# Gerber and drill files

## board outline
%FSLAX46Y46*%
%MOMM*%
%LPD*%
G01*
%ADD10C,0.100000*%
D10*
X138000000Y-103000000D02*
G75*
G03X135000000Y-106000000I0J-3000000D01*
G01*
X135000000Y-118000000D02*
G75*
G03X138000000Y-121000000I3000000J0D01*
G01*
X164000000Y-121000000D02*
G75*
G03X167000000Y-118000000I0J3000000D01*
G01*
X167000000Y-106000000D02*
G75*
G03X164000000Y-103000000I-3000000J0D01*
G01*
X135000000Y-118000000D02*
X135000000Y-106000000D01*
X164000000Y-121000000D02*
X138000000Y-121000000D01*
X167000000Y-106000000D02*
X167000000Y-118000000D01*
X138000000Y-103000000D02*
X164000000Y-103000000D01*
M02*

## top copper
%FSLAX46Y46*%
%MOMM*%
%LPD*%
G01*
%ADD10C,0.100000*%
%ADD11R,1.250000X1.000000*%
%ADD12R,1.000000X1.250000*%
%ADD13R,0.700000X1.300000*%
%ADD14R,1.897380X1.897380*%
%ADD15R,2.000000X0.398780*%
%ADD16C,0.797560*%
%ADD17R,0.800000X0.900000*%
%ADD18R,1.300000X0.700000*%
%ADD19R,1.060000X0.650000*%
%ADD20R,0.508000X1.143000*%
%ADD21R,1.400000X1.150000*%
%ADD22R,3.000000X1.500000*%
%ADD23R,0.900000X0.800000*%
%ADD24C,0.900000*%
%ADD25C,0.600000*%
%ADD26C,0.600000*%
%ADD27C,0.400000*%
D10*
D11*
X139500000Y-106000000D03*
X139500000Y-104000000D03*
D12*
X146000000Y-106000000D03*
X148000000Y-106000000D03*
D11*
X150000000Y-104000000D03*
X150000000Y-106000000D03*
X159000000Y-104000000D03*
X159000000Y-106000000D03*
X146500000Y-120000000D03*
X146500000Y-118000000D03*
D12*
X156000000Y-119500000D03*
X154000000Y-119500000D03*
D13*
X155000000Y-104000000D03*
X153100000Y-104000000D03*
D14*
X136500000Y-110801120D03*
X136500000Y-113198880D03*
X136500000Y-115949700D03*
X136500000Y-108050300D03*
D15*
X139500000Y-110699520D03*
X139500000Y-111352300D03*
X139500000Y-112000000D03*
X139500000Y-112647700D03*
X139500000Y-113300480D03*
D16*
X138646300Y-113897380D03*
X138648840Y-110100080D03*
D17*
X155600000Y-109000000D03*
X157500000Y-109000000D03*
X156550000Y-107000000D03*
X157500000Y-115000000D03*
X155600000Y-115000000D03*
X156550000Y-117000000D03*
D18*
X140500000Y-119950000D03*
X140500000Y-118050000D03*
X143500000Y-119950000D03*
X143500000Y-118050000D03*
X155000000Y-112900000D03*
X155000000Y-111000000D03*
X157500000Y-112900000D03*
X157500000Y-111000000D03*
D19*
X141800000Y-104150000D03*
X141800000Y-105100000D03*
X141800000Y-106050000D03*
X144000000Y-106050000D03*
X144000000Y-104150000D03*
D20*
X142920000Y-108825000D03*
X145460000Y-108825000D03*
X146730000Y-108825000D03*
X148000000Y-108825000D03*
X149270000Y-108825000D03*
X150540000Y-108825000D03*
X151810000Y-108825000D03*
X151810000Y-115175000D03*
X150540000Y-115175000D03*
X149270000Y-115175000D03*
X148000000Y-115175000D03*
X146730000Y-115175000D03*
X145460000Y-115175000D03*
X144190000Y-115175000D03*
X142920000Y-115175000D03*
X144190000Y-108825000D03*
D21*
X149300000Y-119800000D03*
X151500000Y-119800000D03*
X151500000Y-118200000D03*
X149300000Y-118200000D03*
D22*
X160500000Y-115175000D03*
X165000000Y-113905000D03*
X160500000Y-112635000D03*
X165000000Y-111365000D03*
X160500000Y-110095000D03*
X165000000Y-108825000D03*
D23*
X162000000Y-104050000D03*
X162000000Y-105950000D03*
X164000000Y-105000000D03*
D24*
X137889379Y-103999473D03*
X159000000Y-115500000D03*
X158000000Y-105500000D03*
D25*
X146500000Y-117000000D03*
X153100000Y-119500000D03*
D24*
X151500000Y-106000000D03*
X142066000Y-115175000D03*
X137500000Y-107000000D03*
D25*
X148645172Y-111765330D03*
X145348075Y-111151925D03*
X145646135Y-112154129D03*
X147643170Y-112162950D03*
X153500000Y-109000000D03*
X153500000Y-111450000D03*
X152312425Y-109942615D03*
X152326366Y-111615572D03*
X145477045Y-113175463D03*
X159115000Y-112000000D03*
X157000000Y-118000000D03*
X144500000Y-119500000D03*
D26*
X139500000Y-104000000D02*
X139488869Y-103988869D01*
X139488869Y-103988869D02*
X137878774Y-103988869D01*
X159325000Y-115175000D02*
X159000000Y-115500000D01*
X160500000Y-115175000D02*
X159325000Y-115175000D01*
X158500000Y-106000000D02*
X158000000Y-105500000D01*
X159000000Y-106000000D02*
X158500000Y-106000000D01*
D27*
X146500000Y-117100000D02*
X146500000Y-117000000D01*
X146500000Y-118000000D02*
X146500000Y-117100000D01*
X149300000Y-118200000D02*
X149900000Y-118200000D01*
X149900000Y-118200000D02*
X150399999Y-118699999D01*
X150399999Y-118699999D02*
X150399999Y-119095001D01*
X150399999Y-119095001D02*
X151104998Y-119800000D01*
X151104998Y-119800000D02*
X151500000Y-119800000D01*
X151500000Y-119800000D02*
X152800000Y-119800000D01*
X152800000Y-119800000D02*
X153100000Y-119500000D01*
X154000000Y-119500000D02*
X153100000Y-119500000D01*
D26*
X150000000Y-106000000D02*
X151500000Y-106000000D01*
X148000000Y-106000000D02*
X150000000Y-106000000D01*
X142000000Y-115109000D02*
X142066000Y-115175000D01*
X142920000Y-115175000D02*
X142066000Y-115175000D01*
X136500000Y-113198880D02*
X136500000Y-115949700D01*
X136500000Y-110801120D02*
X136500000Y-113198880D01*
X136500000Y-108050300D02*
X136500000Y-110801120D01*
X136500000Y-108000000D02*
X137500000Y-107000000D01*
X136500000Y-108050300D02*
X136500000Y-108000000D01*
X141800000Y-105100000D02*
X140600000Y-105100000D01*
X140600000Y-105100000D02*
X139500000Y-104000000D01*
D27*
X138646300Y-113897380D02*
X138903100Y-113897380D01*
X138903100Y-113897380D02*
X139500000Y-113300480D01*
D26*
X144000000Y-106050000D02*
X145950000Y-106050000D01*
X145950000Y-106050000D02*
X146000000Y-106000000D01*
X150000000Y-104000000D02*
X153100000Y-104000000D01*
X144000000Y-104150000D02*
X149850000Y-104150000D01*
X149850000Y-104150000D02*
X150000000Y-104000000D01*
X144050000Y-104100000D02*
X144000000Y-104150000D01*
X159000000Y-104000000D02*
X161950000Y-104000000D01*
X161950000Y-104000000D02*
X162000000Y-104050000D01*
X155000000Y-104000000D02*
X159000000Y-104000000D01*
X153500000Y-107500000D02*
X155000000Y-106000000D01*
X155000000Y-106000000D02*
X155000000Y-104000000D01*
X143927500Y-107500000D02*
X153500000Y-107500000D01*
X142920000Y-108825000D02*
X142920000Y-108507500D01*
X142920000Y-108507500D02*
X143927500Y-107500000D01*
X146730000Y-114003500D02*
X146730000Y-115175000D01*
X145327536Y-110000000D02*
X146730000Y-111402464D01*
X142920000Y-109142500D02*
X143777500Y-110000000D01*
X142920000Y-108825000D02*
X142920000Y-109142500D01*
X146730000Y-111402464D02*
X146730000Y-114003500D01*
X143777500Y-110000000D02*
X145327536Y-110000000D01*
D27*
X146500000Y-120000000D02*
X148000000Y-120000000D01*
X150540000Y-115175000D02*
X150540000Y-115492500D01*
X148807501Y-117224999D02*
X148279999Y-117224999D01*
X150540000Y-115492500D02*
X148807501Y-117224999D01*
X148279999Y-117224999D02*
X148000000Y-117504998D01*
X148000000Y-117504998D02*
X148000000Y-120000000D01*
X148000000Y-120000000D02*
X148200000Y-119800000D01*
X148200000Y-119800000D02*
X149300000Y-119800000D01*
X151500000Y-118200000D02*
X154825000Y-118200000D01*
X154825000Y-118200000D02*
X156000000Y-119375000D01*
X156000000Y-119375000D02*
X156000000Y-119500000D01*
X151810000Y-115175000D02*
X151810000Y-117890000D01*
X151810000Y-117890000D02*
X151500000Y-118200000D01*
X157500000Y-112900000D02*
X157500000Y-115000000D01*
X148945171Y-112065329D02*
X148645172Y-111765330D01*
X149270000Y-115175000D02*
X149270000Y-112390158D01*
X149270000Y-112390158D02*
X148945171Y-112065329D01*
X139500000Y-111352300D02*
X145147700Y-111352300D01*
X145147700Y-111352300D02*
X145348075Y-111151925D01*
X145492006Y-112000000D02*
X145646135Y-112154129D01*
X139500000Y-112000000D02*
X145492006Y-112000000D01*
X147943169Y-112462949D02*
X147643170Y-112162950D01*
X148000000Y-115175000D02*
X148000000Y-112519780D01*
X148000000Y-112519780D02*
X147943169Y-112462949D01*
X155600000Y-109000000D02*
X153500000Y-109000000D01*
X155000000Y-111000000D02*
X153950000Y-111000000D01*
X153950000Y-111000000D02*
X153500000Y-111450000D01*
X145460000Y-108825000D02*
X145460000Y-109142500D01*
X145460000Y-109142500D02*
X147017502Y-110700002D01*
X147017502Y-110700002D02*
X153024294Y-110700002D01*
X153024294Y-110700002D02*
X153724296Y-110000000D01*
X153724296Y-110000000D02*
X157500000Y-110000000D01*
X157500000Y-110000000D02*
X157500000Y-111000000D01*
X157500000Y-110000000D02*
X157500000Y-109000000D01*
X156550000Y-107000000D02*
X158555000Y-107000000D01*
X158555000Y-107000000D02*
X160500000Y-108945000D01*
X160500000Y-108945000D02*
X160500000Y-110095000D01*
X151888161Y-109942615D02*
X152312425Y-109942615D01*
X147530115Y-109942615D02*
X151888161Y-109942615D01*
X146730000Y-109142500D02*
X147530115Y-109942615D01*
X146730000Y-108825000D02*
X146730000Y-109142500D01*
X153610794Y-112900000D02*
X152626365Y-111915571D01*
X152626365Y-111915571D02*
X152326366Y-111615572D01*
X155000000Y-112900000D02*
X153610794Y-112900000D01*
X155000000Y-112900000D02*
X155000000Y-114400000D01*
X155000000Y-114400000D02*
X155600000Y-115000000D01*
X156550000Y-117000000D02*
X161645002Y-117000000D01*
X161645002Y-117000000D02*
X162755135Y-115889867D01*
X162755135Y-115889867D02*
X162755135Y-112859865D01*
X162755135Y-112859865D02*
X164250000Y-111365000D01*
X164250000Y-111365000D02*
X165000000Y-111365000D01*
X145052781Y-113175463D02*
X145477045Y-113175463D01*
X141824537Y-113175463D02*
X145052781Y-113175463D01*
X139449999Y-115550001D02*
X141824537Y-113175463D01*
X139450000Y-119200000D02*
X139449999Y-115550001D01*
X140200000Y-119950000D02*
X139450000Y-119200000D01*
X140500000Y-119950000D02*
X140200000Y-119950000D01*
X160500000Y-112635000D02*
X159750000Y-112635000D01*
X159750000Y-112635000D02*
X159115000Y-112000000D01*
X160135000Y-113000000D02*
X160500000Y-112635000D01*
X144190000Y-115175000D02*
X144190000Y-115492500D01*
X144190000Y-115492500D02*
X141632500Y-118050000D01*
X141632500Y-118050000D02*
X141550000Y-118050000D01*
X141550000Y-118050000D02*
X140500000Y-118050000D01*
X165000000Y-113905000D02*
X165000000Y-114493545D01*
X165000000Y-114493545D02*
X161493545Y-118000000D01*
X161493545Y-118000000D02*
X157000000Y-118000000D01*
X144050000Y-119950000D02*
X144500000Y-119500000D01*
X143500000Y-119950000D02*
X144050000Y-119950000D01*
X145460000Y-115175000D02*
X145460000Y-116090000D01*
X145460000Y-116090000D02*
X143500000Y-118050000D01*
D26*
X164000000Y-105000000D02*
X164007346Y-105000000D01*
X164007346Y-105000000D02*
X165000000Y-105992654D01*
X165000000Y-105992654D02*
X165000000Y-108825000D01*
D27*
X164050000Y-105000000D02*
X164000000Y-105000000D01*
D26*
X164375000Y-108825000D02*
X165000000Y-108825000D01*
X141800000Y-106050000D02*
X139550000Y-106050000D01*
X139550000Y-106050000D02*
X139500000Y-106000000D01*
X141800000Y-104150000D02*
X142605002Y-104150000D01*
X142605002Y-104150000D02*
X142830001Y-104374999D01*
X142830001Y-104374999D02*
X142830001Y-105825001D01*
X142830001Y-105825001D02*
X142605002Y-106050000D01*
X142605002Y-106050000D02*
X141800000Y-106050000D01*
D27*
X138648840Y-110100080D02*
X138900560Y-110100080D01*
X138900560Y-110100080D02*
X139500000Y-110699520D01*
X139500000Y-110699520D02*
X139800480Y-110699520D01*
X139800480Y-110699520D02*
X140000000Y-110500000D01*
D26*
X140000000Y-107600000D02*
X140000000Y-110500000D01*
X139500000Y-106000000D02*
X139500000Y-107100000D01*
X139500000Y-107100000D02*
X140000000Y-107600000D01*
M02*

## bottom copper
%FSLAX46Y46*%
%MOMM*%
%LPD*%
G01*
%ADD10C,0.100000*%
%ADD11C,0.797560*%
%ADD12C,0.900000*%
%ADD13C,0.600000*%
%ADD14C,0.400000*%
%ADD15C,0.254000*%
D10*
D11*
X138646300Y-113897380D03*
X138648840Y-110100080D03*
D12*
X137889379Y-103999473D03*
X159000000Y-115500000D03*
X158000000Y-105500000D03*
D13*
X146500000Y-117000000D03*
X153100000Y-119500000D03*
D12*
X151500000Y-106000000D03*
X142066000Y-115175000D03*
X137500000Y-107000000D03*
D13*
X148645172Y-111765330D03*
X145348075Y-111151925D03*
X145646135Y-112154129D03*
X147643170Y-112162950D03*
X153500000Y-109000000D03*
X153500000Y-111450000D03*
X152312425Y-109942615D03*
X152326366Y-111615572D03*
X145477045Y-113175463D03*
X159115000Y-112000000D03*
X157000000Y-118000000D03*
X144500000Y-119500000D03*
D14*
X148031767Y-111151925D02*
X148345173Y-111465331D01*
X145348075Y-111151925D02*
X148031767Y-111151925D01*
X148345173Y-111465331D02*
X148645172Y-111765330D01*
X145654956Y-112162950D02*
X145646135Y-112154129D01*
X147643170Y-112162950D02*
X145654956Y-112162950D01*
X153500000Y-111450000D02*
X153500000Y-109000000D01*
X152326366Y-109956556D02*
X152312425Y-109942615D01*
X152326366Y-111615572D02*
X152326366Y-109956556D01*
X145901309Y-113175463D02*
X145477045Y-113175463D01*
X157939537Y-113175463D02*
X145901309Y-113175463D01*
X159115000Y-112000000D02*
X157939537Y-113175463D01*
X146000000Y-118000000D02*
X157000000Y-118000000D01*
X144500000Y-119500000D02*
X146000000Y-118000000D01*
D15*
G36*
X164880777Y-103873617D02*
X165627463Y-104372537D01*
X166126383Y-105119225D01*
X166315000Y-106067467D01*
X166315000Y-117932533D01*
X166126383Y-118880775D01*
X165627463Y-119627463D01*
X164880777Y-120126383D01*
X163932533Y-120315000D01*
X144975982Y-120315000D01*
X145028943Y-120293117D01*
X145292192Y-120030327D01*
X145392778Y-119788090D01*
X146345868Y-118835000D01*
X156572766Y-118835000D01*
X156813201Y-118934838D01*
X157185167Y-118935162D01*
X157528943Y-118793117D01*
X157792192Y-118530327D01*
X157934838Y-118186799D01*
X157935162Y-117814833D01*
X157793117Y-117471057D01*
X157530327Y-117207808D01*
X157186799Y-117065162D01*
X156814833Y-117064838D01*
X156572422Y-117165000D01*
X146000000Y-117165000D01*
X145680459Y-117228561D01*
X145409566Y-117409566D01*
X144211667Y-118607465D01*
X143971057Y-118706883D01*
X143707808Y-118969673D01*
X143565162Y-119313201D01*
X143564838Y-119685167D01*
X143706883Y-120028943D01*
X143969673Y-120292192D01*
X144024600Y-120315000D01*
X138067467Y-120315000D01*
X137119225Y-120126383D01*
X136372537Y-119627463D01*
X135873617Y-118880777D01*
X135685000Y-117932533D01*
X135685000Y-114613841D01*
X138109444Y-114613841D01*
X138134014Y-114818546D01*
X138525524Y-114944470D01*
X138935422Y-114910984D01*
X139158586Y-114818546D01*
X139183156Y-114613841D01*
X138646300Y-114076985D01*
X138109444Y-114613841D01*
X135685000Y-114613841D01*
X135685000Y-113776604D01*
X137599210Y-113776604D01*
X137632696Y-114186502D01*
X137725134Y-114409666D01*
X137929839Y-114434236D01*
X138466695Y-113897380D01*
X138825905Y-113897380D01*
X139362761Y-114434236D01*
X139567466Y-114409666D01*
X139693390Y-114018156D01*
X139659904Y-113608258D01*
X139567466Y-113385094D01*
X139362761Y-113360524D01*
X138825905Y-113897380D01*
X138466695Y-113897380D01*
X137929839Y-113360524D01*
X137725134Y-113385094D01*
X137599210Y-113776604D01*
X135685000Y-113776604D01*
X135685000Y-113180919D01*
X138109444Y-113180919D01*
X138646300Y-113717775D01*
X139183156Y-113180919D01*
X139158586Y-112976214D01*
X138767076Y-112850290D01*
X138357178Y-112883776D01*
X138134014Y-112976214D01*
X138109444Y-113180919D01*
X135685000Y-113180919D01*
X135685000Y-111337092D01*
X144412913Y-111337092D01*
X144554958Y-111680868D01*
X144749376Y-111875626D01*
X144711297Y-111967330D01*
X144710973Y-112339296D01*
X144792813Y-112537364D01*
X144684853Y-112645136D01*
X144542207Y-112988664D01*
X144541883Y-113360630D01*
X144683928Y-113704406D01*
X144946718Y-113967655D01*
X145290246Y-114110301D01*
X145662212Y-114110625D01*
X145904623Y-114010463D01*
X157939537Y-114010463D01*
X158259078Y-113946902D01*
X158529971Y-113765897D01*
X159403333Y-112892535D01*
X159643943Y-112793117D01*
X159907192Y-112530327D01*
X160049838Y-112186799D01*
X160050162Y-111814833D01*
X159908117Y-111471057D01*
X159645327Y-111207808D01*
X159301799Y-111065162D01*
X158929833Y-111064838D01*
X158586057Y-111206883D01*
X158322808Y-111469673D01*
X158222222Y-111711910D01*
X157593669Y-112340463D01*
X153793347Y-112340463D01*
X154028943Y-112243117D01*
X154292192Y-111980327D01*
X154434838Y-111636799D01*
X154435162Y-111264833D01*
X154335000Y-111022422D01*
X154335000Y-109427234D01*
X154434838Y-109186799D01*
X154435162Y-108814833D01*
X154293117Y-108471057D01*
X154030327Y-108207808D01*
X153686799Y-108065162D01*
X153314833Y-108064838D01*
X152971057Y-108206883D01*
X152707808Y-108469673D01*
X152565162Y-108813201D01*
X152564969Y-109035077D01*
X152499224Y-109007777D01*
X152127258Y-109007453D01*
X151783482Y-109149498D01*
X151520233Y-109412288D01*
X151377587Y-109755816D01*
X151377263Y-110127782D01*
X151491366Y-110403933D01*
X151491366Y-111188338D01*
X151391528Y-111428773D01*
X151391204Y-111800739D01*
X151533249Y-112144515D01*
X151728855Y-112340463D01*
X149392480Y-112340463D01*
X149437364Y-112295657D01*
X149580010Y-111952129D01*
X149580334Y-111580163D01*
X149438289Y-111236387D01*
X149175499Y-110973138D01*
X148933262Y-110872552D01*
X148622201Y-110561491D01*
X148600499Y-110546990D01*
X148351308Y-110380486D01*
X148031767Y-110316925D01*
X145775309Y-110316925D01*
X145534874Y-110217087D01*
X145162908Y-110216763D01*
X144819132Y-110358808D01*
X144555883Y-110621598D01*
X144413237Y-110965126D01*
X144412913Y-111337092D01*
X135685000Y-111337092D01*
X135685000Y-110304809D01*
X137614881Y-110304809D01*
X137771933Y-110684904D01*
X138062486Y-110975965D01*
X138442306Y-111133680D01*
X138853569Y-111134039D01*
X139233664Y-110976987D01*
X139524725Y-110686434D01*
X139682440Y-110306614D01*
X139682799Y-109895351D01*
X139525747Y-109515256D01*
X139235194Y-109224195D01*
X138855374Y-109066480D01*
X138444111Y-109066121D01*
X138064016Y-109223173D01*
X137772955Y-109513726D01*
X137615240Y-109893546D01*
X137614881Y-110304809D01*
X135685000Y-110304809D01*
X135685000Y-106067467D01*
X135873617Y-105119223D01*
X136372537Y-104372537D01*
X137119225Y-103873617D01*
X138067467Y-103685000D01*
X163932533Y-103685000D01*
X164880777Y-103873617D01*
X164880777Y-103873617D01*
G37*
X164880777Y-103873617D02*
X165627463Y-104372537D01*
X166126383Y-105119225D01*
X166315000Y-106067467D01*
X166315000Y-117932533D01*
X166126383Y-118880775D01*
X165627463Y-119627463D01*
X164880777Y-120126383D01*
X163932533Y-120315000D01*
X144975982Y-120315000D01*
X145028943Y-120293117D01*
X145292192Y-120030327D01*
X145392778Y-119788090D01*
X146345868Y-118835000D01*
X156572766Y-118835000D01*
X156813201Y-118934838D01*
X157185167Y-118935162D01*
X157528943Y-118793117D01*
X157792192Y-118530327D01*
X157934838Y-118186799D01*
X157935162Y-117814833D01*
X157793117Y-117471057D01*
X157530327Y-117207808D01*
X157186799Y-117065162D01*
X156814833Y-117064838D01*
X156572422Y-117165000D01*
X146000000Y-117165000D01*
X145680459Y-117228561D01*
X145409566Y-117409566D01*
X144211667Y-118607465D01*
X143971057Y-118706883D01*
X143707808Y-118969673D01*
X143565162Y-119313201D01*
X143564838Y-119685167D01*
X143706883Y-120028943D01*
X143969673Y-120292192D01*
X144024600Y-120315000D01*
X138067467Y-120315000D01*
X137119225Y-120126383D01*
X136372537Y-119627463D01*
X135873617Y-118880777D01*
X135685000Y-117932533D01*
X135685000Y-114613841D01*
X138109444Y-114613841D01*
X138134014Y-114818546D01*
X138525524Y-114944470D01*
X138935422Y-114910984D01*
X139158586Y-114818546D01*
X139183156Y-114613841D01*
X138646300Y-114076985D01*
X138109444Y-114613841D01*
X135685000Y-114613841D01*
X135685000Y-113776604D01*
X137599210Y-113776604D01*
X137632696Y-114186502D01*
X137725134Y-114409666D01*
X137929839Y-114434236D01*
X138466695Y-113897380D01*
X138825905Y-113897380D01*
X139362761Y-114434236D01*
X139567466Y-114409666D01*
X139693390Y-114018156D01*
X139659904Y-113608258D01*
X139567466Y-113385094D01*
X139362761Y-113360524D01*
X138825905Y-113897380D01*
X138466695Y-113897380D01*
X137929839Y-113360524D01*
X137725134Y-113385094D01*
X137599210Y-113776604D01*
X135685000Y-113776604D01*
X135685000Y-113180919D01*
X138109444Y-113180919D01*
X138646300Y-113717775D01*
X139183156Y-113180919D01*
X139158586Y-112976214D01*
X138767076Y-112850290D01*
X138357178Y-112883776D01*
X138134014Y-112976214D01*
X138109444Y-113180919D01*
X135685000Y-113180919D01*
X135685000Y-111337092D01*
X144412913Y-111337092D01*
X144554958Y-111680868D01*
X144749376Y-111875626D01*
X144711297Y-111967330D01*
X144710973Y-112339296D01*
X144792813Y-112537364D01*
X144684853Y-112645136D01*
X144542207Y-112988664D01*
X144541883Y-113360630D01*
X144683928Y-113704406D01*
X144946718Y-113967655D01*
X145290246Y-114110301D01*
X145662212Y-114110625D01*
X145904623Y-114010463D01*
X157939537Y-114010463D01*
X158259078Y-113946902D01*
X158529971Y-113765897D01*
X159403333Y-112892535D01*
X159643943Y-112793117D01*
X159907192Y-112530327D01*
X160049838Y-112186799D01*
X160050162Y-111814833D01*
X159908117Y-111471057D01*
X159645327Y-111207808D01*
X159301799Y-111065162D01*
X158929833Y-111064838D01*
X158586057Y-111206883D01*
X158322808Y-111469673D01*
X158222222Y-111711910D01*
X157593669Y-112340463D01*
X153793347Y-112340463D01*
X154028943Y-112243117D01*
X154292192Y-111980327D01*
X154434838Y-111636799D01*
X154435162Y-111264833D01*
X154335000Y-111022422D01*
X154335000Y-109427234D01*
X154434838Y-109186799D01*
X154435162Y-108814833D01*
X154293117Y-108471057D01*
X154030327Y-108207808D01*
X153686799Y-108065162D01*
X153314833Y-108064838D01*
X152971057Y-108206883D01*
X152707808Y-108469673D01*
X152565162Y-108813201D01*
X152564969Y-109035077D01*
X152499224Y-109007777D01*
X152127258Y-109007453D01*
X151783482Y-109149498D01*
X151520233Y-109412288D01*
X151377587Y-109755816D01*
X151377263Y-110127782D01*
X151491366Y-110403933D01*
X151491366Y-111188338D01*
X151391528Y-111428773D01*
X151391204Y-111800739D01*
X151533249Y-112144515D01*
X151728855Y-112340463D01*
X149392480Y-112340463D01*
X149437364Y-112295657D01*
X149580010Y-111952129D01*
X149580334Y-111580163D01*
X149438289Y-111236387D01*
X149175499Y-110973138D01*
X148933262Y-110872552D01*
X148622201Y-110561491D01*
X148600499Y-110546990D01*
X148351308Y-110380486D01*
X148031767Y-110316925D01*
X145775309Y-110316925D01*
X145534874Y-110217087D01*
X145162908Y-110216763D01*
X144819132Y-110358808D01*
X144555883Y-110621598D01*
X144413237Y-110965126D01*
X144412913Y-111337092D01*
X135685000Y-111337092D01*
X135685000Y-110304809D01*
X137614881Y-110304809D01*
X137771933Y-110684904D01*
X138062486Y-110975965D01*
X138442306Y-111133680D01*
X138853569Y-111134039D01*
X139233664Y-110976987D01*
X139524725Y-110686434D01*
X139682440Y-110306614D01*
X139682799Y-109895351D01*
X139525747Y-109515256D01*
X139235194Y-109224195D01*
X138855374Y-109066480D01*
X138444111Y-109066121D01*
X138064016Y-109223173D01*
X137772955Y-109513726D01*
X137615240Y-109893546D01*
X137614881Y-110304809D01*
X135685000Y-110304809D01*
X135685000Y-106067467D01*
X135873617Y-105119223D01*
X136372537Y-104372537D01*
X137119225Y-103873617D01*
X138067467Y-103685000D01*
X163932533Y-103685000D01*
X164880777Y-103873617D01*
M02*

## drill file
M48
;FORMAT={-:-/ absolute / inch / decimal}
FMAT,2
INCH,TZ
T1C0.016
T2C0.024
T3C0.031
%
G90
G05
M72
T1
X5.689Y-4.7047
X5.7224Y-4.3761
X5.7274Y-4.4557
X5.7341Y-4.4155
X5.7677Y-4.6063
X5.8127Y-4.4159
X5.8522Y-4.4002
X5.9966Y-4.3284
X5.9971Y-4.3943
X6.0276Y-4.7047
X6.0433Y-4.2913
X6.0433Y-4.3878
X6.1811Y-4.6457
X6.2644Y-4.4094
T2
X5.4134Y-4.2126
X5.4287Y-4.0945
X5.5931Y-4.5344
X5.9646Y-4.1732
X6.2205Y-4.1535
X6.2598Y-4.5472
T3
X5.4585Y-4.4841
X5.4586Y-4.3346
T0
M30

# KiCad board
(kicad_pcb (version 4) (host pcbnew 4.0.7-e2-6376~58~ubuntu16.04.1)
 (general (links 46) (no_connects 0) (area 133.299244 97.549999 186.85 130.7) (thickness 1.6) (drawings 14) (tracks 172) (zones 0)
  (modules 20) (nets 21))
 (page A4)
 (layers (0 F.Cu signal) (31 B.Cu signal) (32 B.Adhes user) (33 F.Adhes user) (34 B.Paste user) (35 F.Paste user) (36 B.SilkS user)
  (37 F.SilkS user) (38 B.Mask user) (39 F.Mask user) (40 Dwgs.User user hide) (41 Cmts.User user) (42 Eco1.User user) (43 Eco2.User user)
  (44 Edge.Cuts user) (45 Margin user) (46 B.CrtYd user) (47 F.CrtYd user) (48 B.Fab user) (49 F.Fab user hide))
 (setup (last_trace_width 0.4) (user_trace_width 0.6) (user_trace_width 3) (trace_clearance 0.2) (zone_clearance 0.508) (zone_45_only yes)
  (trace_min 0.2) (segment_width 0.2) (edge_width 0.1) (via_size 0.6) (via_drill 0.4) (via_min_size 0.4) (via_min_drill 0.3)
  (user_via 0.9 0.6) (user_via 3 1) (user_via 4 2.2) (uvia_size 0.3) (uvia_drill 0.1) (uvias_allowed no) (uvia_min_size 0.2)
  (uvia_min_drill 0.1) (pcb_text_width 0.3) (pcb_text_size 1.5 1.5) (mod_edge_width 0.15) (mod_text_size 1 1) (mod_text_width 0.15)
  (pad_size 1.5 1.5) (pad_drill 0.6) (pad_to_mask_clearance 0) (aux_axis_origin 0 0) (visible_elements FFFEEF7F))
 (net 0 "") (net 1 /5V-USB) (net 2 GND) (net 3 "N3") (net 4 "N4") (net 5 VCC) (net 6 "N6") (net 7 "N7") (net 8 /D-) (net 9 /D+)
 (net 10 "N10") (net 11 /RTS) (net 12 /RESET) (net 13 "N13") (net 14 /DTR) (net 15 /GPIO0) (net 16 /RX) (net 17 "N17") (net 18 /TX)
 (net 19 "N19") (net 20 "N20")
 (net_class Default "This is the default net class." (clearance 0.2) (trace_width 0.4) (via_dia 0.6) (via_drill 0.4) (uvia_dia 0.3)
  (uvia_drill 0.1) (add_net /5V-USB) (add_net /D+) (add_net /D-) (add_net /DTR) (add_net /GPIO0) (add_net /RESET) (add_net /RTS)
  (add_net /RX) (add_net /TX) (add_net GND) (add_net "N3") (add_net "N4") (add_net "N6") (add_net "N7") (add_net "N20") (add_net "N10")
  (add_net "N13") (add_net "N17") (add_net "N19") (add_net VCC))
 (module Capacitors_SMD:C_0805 (layer F.Cu) (at 139.5 105 90)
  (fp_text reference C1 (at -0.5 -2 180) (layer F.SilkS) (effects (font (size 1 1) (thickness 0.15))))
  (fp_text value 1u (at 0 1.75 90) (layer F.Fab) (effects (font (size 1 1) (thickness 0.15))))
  (pad 1 smd rect (at -1 0 90) (size 1 1.25) (layers F.Cu F.Paste F.Mask) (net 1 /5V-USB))
  (pad 2 smd rect (at 1 0 90) (size 1 1.25) (layers F.Cu F.Paste F.Mask) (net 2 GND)))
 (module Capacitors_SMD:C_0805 (layer F.Cu) (at 147 106)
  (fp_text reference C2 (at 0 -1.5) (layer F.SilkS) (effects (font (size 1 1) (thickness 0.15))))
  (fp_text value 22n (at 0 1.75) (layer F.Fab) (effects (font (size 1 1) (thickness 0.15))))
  (pad 1 smd rect (at -1 0) (size 1 1.25) (layers F.Cu F.Paste F.Mask) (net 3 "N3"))
  (pad 2 smd rect (at 1 0) (size 1 1.25) (layers F.Cu F.Paste F.Mask) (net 2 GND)))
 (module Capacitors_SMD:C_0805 (layer F.Cu) (at 150 105 270)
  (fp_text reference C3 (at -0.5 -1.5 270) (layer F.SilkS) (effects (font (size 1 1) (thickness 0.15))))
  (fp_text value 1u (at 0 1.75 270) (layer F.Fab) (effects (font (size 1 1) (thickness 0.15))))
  (pad 1 smd rect (at -1 0 270) (size 1 1.25) (layers F.Cu F.Paste F.Mask) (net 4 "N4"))
  (pad 2 smd rect (at 1 0 270) (size 1 1.25) (layers F.Cu F.Paste F.Mask) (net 2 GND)))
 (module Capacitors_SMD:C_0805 (layer F.Cu) (at 159 105 270)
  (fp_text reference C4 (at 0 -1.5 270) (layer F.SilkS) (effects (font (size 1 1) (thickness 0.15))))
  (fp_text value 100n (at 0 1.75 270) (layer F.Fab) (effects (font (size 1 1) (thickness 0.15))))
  (pad 1 smd rect (at -1 0 270) (size 1 1.25) (layers F.Cu F.Paste F.Mask) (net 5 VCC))
  (pad 2 smd rect (at 1 0 270) (size 1 1.25) (layers F.Cu F.Paste F.Mask) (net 2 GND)))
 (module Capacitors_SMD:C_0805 (layer F.Cu) (at 146.5 119 90)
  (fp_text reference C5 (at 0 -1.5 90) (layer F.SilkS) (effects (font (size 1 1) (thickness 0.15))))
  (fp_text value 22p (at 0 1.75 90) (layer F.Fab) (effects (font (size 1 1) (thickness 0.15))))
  (pad 1 smd rect (at -1 0 90) (size 1 1.25) (layers F.Cu F.Paste F.Mask) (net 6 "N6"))
  (pad 2 smd rect (at 1 0 90) (size 1 1.25) (layers F.Cu F.Paste F.Mask) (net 2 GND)))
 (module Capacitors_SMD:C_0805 (layer F.Cu) (at 155 119.5 180)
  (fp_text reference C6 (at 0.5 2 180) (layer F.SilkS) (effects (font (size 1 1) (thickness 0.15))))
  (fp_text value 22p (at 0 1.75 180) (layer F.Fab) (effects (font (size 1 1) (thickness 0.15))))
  (pad 1 smd rect (at -1 0 180) (size 1 1.25) (layers F.Cu F.Paste F.Mask) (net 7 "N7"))
  (pad 2 smd rect (at 1 0 180) (size 1 1.25) (layers F.Cu F.Paste F.Mask) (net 2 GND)))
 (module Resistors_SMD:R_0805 (layer F.Cu) (at 154.05 104 180)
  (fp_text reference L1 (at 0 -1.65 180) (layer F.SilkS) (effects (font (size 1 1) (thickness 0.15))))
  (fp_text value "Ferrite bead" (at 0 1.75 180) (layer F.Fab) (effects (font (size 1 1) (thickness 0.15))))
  (pad 1 smd rect (at -0.95 0 180) (size 0.7 1.3) (layers F.Cu F.Paste F.Mask) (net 5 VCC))
  (pad 2 smd rect (at 0.95 0 180) (size 0.7 1.3) (layers F.Cu F.Paste F.Mask) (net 4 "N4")))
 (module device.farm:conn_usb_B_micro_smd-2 (layer F.Cu) (at 136.5 112 270)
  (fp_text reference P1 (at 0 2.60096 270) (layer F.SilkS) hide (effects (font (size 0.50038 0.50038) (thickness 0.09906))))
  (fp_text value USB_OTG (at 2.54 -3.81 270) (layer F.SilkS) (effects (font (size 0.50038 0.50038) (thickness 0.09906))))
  (pad 6 smd rect (at -1.19888 0 270) (size 1.89738 1.89738) (layers F.Cu F.Paste F.Mask) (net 2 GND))
  (pad 6 smd rect (at 1.19888 0 270) (size 1.89738 1.89738) (layers F.Cu F.Paste F.Mask) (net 2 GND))
  (pad 6 smd rect (at 3.9497 0 270) (size 1.89738 1.89738) (layers F.Cu F.Paste F.Mask) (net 2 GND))
  (pad 6 smd rect (at -3.9497 0 270) (size 1.89738 1.89738) (layers F.Cu F.Paste F.Mask) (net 2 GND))
  (pad 1 smd rect (at -1.30048 -3 270) (size 0.39878 2) (layers F.Cu F.Paste F.Mask) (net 1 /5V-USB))
  (pad 2 smd rect (at -0.6477 -3 270) (size 0.39878 2) (layers F.Cu F.Paste F.Mask) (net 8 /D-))
  (pad 3 smd rect (at 0 -3 270) (size 0.39878 2) (layers F.Cu F.Paste F.Mask) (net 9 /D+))
  (pad 4 smd rect (at 0.6477 -3 270) (size 0.39878 2) (layers F.Cu F.Paste F.Mask))
  (pad 5 smd rect (at 1.30048 -3 270) (size 0.39878 2) (layers F.Cu F.Paste F.Mask) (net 2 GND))
  (pad 5 thru_hole circle (at 1.89738 -2.1463 270) (size 0.79756 0.79756) (drill 0.79756) (layers *.Cu *.Mask F.SilkS) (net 2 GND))
  (pad 1 thru_hole circle (at -1.89992 -2.14884 270) (size 0.79756 0.79756) (drill 0.79756) (layers *.Cu *.Mask F.SilkS) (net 1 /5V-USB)))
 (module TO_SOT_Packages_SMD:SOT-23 (layer F.Cu) (at 156.55 108 90)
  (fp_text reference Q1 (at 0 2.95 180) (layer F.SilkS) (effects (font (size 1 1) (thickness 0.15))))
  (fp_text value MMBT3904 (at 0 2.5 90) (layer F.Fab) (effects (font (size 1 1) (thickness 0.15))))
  (pad 1 smd rect (at -1 -0.95 90) (size 0.9 0.8) (layers F.Cu F.Paste F.Mask) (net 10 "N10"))
  (pad 2 smd rect (at -1 0.95 90) (size 0.9 0.8) (layers F.Cu F.Paste F.Mask) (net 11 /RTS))
  (pad 3 smd rect (at 1 0 90) (size 0.9 0.8) (layers F.Cu F.Paste F.Mask) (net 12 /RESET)))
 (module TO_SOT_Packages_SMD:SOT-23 (layer F.Cu) (at 156.55 116 270)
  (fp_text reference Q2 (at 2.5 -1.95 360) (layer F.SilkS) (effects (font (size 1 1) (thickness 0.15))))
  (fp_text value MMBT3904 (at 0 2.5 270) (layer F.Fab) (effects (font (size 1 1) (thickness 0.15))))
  (pad 1 smd rect (at -1 -0.95 270) (size 0.9 0.8) (layers F.Cu F.Paste F.Mask) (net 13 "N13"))
  (pad 2 smd rect (at -1 0.95 270) (size 0.9 0.8) (layers F.Cu F.Paste F.Mask) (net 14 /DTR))
  (pad 3 smd rect (at 1 0 270) (size 0.9 0.8) (layers F.Cu F.Paste F.Mask) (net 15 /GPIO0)))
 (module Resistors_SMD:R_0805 (layer F.Cu) (at 140.5 119 90)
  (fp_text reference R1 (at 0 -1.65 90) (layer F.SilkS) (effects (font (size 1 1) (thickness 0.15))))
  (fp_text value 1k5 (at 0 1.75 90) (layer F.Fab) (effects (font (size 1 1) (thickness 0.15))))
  (pad 1 smd rect (at -0.95 0 90) (size 0.7 1.3) (layers F.Cu F.Paste F.Mask) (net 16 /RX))
  (pad 2 smd rect (at 0.95 0 90) (size 0.7 1.3) (layers F.Cu F.Paste F.Mask) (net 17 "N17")))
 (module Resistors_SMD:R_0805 (layer F.Cu) (at 143.5 119 90)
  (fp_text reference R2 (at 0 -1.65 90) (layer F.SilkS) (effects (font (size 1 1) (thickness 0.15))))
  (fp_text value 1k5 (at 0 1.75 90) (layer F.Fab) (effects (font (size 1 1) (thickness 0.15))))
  (pad 1 smd rect (at -0.95 0 90) (size 0.7 1.3) (layers F.Cu F.Paste F.Mask) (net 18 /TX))
  (pad 2 smd rect (at 0.95 0 90) (size 0.7 1.3) (layers F.Cu F.Paste F.Mask) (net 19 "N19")))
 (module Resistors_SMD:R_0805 (layer F.Cu) (at 155 111.95 90)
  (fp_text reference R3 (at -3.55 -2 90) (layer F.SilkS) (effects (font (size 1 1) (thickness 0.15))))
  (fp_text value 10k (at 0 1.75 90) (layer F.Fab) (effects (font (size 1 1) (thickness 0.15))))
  (pad 1 smd rect (at -0.95 0 90) (size 0.7 1.3) (layers F.Cu F.Paste F.Mask) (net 14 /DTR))
  (pad 2 smd rect (at 0.95 0 90) (size 0.7 1.3) (layers F.Cu F.Paste F.Mask) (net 10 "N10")))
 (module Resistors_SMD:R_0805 (layer F.Cu) (at 157.5 111.95 90)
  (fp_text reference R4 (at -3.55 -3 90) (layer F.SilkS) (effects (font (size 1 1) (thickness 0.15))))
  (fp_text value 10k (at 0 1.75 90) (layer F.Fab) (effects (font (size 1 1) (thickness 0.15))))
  (pad 1 smd rect (at -0.95 0 90) (size 0.7 1.3) (layers F.Cu F.Paste F.Mask) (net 13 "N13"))
  (pad 2 smd rect (at 0.95 0 90) (size 0.7 1.3) (layers F.Cu F.Paste F.Mask) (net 11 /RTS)))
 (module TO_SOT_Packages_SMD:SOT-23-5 (layer F.Cu) (at 142.9 105.1)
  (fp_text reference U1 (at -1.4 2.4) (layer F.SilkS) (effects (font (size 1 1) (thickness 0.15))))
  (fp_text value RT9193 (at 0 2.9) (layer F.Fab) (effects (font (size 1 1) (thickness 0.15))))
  (pad 1 smd rect (at -1.1 -0.95) (size 1.06 0.65) (layers F.Cu F.Paste F.Mask) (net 1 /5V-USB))
  (pad 2 smd rect (at -1.1 0) (size 1.06 0.65) (layers F.Cu F.Paste F.Mask) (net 2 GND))
  (pad 3 smd rect (at -1.1 0.95) (size 1.06 0.65) (layers F.Cu F.Paste F.Mask) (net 1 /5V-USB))
  (pad 4 smd rect (at 1.1 0.95) (size 1.06 0.65) (layers F.Cu F.Paste F.Mask) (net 3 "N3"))
  (pad 5 smd rect (at 1.1 -0.95) (size 1.06 0.65) (layers F.Cu F.Paste F.Mask) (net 4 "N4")))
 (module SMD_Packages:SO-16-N (layer F.Cu) (at 147.365 112)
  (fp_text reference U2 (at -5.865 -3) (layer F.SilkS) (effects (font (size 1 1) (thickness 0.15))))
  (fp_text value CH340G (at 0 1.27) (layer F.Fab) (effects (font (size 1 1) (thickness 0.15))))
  (pad 16 smd rect (at -4.445 -3.175) (size 0.508 1.143) (layers F.Cu F.Paste F.Mask) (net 5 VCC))
  (pad 14 smd rect (at -1.905 -3.175) (size 0.508 1.143) (layers F.Cu F.Paste F.Mask) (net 11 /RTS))
  (pad 13 smd rect (at -0.635 -3.175) (size 0.508 1.143) (layers F.Cu F.Paste F.Mask) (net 14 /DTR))
  (pad 12 smd rect (at 0.635 -3.175) (size 0.508 1.143) (layers F.Cu F.Paste F.Mask))
  (pad 11 smd rect (at 1.905 -3.175) (size 0.508 1.143) (layers F.Cu F.Paste F.Mask))
  (pad 10 smd rect (at 3.175 -3.175) (size 0.508 1.143) (layers F.Cu F.Paste F.Mask))
  (pad 9 smd rect (at 4.445 -3.175) (size 0.508 1.143) (layers F.Cu F.Paste F.Mask))
  (pad 8 smd rect (at 4.445 3.175) (size 0.508 1.143) (layers F.Cu F.Paste F.Mask) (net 7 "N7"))
  (pad 7 smd rect (at 3.175 3.175) (size 0.508 1.143) (layers F.Cu F.Paste F.Mask) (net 6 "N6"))
  (pad 6 smd rect (at 1.905 3.175) (size 0.508 1.143) (layers F.Cu F.Paste F.Mask) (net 8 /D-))
  (pad 5 smd rect (at 0.635 3.175) (size 0.508 1.143) (layers F.Cu F.Paste F.Mask) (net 9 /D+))
  (pad 4 smd rect (at -0.635 3.175) (size 0.508 1.143) (layers F.Cu F.Paste F.Mask) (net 5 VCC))
  (pad 3 smd rect (at -1.905 3.175) (size 0.508 1.143) (layers F.Cu F.Paste F.Mask) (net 19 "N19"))
  (pad 2 smd rect (at -3.175 3.175) (size 0.508 1.143) (layers F.Cu F.Paste F.Mask) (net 17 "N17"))
  (pad 1 smd rect (at -4.445 3.175) (size 0.508 1.143) (layers F.Cu F.Paste F.Mask) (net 2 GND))
  (pad 15 smd rect (at -3.175 -3.175) (size 0.508 1.143) (layers F.Cu F.Paste F.Mask)))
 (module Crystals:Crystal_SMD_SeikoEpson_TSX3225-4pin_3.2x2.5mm (layer F.Cu) (at 150.4 119)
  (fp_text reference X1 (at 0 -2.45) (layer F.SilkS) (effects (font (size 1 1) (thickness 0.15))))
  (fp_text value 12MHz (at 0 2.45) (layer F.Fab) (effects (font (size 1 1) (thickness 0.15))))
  (pad 1 smd rect (at -1.1 0.8) (size 1.4 1.15) (layers F.Cu F.Paste F.Mask) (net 6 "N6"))
  (pad 2 smd rect (at 1.1 0.8) (size 1.4 1.15) (layers F.Cu F.Paste F.Mask) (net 2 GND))
  (pad 3 smd rect (at 1.1 -0.8) (size 1.4 1.15) (layers F.Cu F.Paste F.Mask) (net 7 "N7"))
  (pad 4 smd rect (at -1.1 -0.8) (size 1.4 1.15) (layers F.Cu F.Paste F.Mask) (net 2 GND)))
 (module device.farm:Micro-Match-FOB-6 (layer F.Cu) (at 162.75 112 90)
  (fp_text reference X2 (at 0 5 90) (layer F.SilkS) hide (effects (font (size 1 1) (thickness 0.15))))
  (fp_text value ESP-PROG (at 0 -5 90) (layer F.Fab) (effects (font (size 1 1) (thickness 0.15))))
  (pad 1 smd rect (at -3.175 -2.25 90) (size 1.5 3) (layers F.Cu F.Paste F.Mask) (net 2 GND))
  (pad 2 smd rect (at -1.905 2.25 90) (size 1.5 3) (layers F.Cu F.Paste F.Mask) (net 18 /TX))
  (pad 3 smd rect (at -0.635 -2.25 90) (size 1.5 3) (layers F.Cu F.Paste F.Mask) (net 16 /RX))
  (pad 4 smd rect (at 0.635 2.25 90) (size 1.5 3) (layers F.Cu F.Paste F.Mask) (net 15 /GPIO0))
  (pad 5 smd rect (at 1.905 -2.25 90) (size 1.5 3) (layers F.Cu F.Paste F.Mask) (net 12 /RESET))
  (pad 6 smd rect (at 3.175 2.25 90) (size 1.5 3) (layers F.Cu F.Paste F.Mask) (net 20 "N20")))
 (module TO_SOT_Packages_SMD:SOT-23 (layer F.Cu) (at 163 105)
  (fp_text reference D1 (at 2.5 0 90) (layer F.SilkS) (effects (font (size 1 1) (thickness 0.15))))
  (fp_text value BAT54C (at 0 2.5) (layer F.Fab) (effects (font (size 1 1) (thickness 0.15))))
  (pad 1 smd rect (at -1 -0.95) (size 0.9 0.8) (layers F.Cu F.Paste F.Mask) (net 5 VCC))
  (pad 2 smd rect (at -1 0.95) (size 0.9 0.8) (layers F.Cu F.Paste F.Mask))
  (pad 3 smd rect (at 1 0) (size 0.9 0.8) (layers F.Cu F.Paste F.Mask) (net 20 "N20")))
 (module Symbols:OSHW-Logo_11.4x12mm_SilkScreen (layer B.Cu) (at 152.5 112 90)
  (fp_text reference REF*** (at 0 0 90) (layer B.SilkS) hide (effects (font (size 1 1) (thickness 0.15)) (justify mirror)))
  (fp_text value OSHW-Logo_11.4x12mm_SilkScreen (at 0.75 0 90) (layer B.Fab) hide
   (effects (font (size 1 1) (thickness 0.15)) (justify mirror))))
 (gr_arc (start 138 106) (end 135 106) (angle 90) (layer Edge.Cuts) (width 0.1))
 (gr_arc (start 138 118) (end 138 121) (angle 90) (layer Edge.Cuts) (width 0.1))
 (gr_arc (start 164 118) (end 167 118) (angle 90) (layer Edge.Cuts) (width 0.1))
 (gr_arc (start 164 106) (end 164 103) (angle 90) (layer Edge.Cuts) (width 0.1))
 (gr_line (start 135 118) (end 135 106) (layer Edge.Cuts) (width 0.1))
 (gr_line (start 164 121) (end 138 121) (layer Edge.Cuts) (width 0.1))
 (gr_line (start 167 106) (end 167 118) (layer Edge.Cuts) (width 0.1))
 (gr_line (start 138 103) (end 164 103) (layer Edge.Cuts) (width 0.1))
 (via (at 137.889379 103.999473) (size 0.9) (drill 0.6) (layers F.Cu B.Cu) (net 2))
 (segment (start 139.5 104) (end 139.488869 103.988869) (width 0.6) (layer F.Cu) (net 2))
 (segment (start 139.488869 103.988869) (end 137.878774 103.988869) (width 0.6) (layer F.Cu) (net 2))
 (segment (start 159.325 115.175) (end 159 115.5) (width 0.6) (layer F.Cu) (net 2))
 (via (at 159 115.5) (size 0.9) (drill 0.6) (layers F.Cu B.Cu) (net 2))
 (segment (start 160.5 115.175) (end 159.325 115.175) (width 0.6) (layer F.Cu) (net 2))
 (segment (start 158.5 106) (end 158 105.5) (width 0.6) (layer F.Cu) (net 2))
 (via (at 158 105.5) (size 0.9) (drill 0.6) (layers F.Cu B.Cu) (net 2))
 (segment (start 159 106) (end 158.5 106) (width 0.6) (layer F.Cu) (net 2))
 (segment (start 146.5 117.1) (end 146.5 117) (width 0.4) (layer F.Cu) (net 2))
 (via (at 146.5 117) (size 0.6) (drill 0.4) (layers F.Cu B.Cu) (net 2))
 (segment (start 146.5 118) (end 146.5 117.1) (width 0.4) (layer F.Cu) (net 2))
 (segment (start 149.3 118.2) (end 149.9 118.2) (width 0.4) (layer F.Cu) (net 2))
 (segment (start 149.9 118.2) (end 150.399999 118.699999) (width 0.4) (layer F.Cu) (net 2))
 (segment (start 150.399999 118.699999) (end 150.399999 119.095001) (width 0.4) (layer F.Cu) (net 2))
 (segment (start 150.399999 119.095001) (end 151.104998 119.8) (width 0.4) (layer F.Cu) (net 2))
 (segment (start 151.104998 119.8) (end 151.5 119.8) (width 0.4) (layer F.Cu) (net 2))
 (segment (start 151.5 119.8) (end 152.8 119.8) (width 0.4) (layer F.Cu) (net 2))
 (segment (start 152.8 119.8) (end 153.1 119.5) (width 0.4) (layer F.Cu) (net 2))
 (via (at 153.1 119.5) (size 0.6) (drill 0.4) (layers F.Cu B.Cu) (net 2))
 (segment (start 154 119.5) (end 153.1 119.5) (width 0.4) (layer F.Cu) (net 2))
 (via (at 151.5 106) (size 0.9) (drill 0.6) (layers F.Cu B.Cu) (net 2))
 (segment (start 150 106) (end 151.5 106) (width 0.6) (layer F.Cu) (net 2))
 (segment (start 148 106) (end 150 106) (width 0.6) (layer F.Cu) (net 2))
 (segment (start 142 115.109) (end 142.066 115.175) (width 0.6) (layer F.Cu) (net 2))
 (via (at 142.066 115.175) (size 0.9) (drill 0.6) (layers F.Cu B.Cu) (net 2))
 (segment (start 142.92 115.175) (end 142.066 115.175) (width 0.6) (layer F.Cu) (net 2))
 (segment (start 136.5 113.19888) (end 136.5 115.9497) (width 0.6) (layer F.Cu) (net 2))
 (segment (start 136.5 110.80112) (end 136.5 113.19888) (width 0.6) (layer F.Cu) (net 2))
 (segment (start 136.5 108.0503) (end 136.5 110.80112) (width 0.6) (layer F.Cu) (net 2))
 (segment (start 136.5 108) (end 137.5 107) (width 0.6) (layer F.Cu) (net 2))
 (via (at 137.5 107) (size 0.9) (drill 0.6) (layers F.Cu B.Cu) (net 2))
 (segment (start 136.5 108.0503) (end 136.5 108) (width 0.6) (layer F.Cu) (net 2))
 (segment (start 141.8 105.1) (end 140.6 105.1) (width 0.6) (layer F.Cu) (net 2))
 (segment (start 140.6 105.1) (end 139.5 104) (width 0.6) (layer F.Cu) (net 2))
 (segment (start 138.6463 113.89738) (end 138.9031 113.89738) (width 0.4) (layer F.Cu) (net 2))
 (segment (start 138.9031 113.89738) (end 139.5 113.30048) (width 0.4) (layer F.Cu) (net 2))
 (segment (start 144 106.05) (end 145.95 106.05) (width 0.6) (layer F.Cu) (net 3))
 (segment (start 145.95 106.05) (end 146 106) (width 0.6) (layer F.Cu) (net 3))
 (segment (start 150 104) (end 153.1 104) (width 0.6) (layer F.Cu) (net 4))
 (segment (start 144 104.15) (end 149.85 104.15) (width 0.6) (layer F.Cu) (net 4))
 (segment (start 149.85 104.15) (end 150 104) (width 0.6) (layer F.Cu) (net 4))
 (segment (start 144.05 104.1) (end 144 104.15) (width 0.6) (layer F.Cu) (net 4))
 (segment (start 159 104) (end 161.95 104) (width 0.6) (layer F.Cu) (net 5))
 (segment (start 161.95 104) (end 162 104.05) (width 0.6) (layer F.Cu) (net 5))
 (segment (start 155 104) (end 159 104) (width 0.6) (layer F.Cu) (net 5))
 (segment (start 153.5 107.5) (end 155 106) (width 0.6) (layer F.Cu) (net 5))
 (segment (start 155 106) (end 155 104) (width 0.6) (layer F.Cu) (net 5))
 (segment (start 143.9275 107.5) (end 153.5 107.5) (width 0.6) (layer F.Cu) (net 5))
 (segment (start 142.92 108.825) (end 142.92 108.5075) (width 0.6) (layer F.Cu) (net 5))
 (segment (start 142.92 108.5075) (end 143.9275 107.5) (width 0.6) (layer F.Cu) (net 5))
 (segment (start 146.73 114.0035) (end 146.73 115.175) (width 0.6) (layer F.Cu) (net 5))
 (segment (start 145.327536 110) (end 146.73 111.402464) (width 0.6) (layer F.Cu) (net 5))
 (segment (start 142.92 109.1425) (end 143.7775 110) (width 0.6) (layer F.Cu) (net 5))
 (segment (start 142.92 108.825) (end 142.92 109.1425) (width 0.6) (layer F.Cu) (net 5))
 (segment (start 146.73 111.402464) (end 146.73 114.0035) (width 0.6) (layer F.Cu) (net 5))
 (segment (start 143.7775 110) (end 145.327536 110) (width 0.6) (layer F.Cu) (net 5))
 (segment (start 146.5 120) (end 148 120) (width 0.4) (layer F.Cu) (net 6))
 (segment (start 150.54 115.175) (end 150.54 115.4925) (width 0.4) (layer F.Cu) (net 6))
 (segment (start 148.807501 117.224999) (end 148.279999 117.224999) (width 0.4) (layer F.Cu) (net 6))
 (segment (start 150.54 115.4925) (end 148.807501 117.224999) (width 0.4) (layer F.Cu) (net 6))
 (segment (start 148.279999 117.224999) (end 148 117.504998) (width 0.4) (layer F.Cu) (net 6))
 (segment (start 148 117.504998) (end 148 120) (width 0.4) (layer F.Cu) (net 6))
 (segment (start 148 120) (end 148.2 119.8) (width 0.4) (layer F.Cu) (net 6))
 (segment (start 148.2 119.8) (end 149.3 119.8) (width 0.4) (layer F.Cu) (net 6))
 (segment (start 151.5 118.2) (end 154.825 118.2) (width 0.4) (layer F.Cu) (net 7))
 (segment (start 154.825 118.2) (end 156 119.375) (width 0.4) (layer F.Cu) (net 7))
 (segment (start 156 119.375) (end 156 119.5) (width 0.4) (layer F.Cu) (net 7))
 (segment (start 151.81 115.175) (end 151.81 117.89) (width 0.4) (layer F.Cu) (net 7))
 (segment (start 151.81 117.89) (end 151.5 118.2) (width 0.4) (layer F.Cu) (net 7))
 (segment (start 157.5 112.9) (end 157.5 115) (width 0.4) (layer F.Cu) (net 13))
 (segment (start 148.031767 111.151925) (end 148.345173 111.465331) (width 0.4) (layer B.Cu) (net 8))
 (segment (start 145.348075 111.151925) (end 148.031767 111.151925) (width 0.4) (layer B.Cu) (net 8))
 (segment (start 148.945171 112.065329) (end 148.645172 111.76533) (width 0.4) (layer F.Cu) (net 8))
 (segment (start 149.27 115.175) (end 149.27 112.390158) (width 0.4) (layer F.Cu) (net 8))
 (segment (start 148.345173 111.465331) (end 148.645172 111.76533) (width 0.4) (layer B.Cu) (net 8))
 (segment (start 149.27 112.390158) (end 148.945171 112.065329) (width 0.4) (layer F.Cu) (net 8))
 (via (at 148.645172 111.76533) (size 0.6) (drill 0.4) (layers F.Cu B.Cu) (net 8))
 (segment (start 139.5 111.3523) (end 145.1477 111.3523) (width 0.4) (layer F.Cu) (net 8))
 (via (at 145.348075 111.151925) (size 0.6) (drill 0.4) (layers F.Cu B.Cu) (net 8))
 (segment (start 145.1477 111.3523) (end 145.348075 111.151925) (width 0.4) (layer F.Cu) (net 8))
 (segment (start 145.492006 112) (end 145.646135 112.154129) (width 0.4) (layer F.Cu) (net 9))
 (segment (start 139.5 112) (end 145.492006 112) (width 0.4) (layer F.Cu) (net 9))
 (segment (start 145.654956 112.16295) (end 145.646135 112.154129) (width 0.4) (layer B.Cu) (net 9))
 (segment (start 147.64317 112.16295) (end 145.654956 112.16295) (width 0.4) (layer B.Cu) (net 9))
 (via (at 145.646135 112.154129) (size 0.6) (drill 0.4) (layers F.Cu B.Cu) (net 9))
 (segment (start 147.943169 112.462949) (end 147.64317 112.16295) (width 0.4) (layer F.Cu) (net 9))
 (segment (start 148 115.175) (end 148 112.51978) (width 0.4) (layer F.Cu) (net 9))
 (segment (start 148 112.51978) (end 147.943169 112.462949) (width 0.4) (layer F.Cu) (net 9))
 (via (at 147.64317 112.16295) (size 0.6) (drill 0.4) (layers F.Cu B.Cu) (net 9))
 (segment (start 155.6 109) (end 153.5 109) (width 0.4) (layer F.Cu) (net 10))
 (via (at 153.5 109) (size 0.6) (drill 0.4) (layers F.Cu B.Cu) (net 10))
 (segment (start 153.5 111.45) (end 153.5 109) (width 0.4) (layer B.Cu) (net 10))
 (via (at 153.5 111.45) (size 0.6) (drill 0.4) (layers F.Cu B.Cu) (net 10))
 (segment (start 155 111) (end 153.95 111) (width 0.4) (layer F.Cu) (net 10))
 (segment (start 153.95 111) (end 153.5 111.45) (width 0.4) (layer F.Cu) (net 10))
 (segment (start 145.46 108.825) (end 145.46 109.1425) (width 0.4) (layer F.Cu) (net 11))
 (segment (start 145.46 109.1425) (end 147.017502 110.700002) (width 0.4) (layer F.Cu) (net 11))
 (segment (start 147.017502 110.700002) (end 153.024294 110.700002) (width 0.4) (layer F.Cu) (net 11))
 (segment (start 153.024294 110.700002) (end 153.724296 110) (width 0.4) (layer F.Cu) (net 11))
 (segment (start 153.724296 110) (end 157.5 110) (width 0.4) (layer F.Cu) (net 11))
 (segment (start 157.5 110) (end 157.5 111) (width 0.4) (layer F.Cu) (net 11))
 (segment (start 157.5 110) (end 157.5 109) (width 0.4) (layer F.Cu) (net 11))
 (segment (start 156.55 107) (end 158.555 107) (width 0.4) (layer F.Cu) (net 12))
 (segment (start 158.555 107) (end 160.5 108.945) (width 0.4) (layer F.Cu) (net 12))
 (segment (start 160.5 108.945) (end 160.5 110.095) (width 0.4) (layer F.Cu) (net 12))
 (segment (start 151.888161 109.942615) (end 152.312425 109.942615) (width 0.4) (layer F.Cu) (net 14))
 (segment (start 147.530115 109.942615) (end 151.888161 109.942615) (width 0.4) (layer F.Cu) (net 14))
 (segment (start 146.73 109.1425) (end 147.530115 109.942615) (width 0.4) (layer F.Cu) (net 14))
 (segment (start 146.73 108.825) (end 146.73 109.1425) (width 0.4) (layer F.Cu) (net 14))
 (segment (start 152.326366 109.956556) (end 152.312425 109.942615) (width 0.4) (layer B.Cu) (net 14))
 (segment (start 152.326366 111.615572) (end 152.326366 109.956556) (width 0.4) (layer B.Cu) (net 14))
 (via (at 152.312425 109.942615) (size 0.6) (drill 0.4) (layers F.Cu B.Cu) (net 14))
 (segment (start 153.610794 112.9) (end 152.626365 111.915571) (width 0.4) (layer F.Cu) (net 14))
 (segment (start 152.626365 111.915571) (end 152.326366 111.615572) (width 0.4) (layer F.Cu) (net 14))
 (segment (start 155 112.9) (end 153.610794 112.9) (width 0.4) (layer F.Cu) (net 14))
 (via (at 152.326366 111.615572) (size 0.6) (drill 0.4) (layers F.Cu B.Cu) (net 14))
 (segment (start 155 112.9) (end 155 114.4) (width 0.4) (layer F.Cu) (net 14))
 (segment (start 155 114.4) (end 155.6 115) (width 0.4) (layer F.Cu) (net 14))
 (segment (start 156.55 117) (end 161.645002 117) (width 0.4) (layer F.Cu) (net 15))
 (segment (start 161.645002 117) (end 162.755135 115.889867) (width 0.4) (layer F.Cu) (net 15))
 (segment (start 162.755135 115.889867) (end 162.755135 112.859865) (width 0.4) (layer F.Cu) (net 15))
 (segment (start 162.755135 112.859865) (end 164.25 111.365) (width 0.4) (layer F.Cu) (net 15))
 (segment (start 164.25 111.365) (end 165 111.365) (width 0.4) (layer F.Cu) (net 15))
 (segment (start 145.901309 113.175463) (end 145.477045 113.175463) (width 0.4) (layer B.Cu) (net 16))
 (segment (start 145.052781 113.175463) (end 145.477045 113.175463) (width 0.4) (layer F.Cu) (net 16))
 (segment (start 141.824537 113.175463) (end 145.052781 113.175463) (width 0.4) (layer F.Cu) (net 16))
 (segment (start 157.939537 113.175463) (end 145.901309 113.175463) (width 0.4) (layer B.Cu) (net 16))
 (segment (start 139.449999 115.550001) (end 141.824537 113.175463) (width 0.4) (layer F.Cu) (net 16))
 (segment (start 139.45 119.2) (end 139.449999 115.550001) (width 0.4) (layer F.Cu) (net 16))
 (segment (start 159.115 112) (end 157.939537 113.175463) (width 0.4) (layer B.Cu) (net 16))
 (segment (start 140.2 119.95) (end 139.45 119.2) (width 0.4) (layer F.Cu) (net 16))
 (segment (start 140.5 119.95) (end 140.2 119.95) (width 0.4) (layer F.Cu) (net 16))
 (via (at 145.477045 113.175463) (size 0.6) (drill 0.4) (layers F.Cu B.Cu) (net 16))
 (via (at 159.115 112) (size 0.6) (drill 0.4) (layers F.Cu B.Cu) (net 16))
 (segment (start 160.5 112.635) (end 159.75 112.635) (width 0.4) (layer F.Cu) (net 16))
 (segment (start 159.75 112.635) (end 159.115 112) (width 0.4) (layer F.Cu) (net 16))
 (segment (start 160.135 113) (end 160.5 112.635) (width 0.4) (layer F.Cu) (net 16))
 (segment (start 144.19 115.175) (end 144.19 115.4925) (width 0.4) (layer F.Cu) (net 17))
 (segment (start 144.19 115.4925) (end 141.6325 118.05) (width 0.4) (layer F.Cu) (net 17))
 (segment (start 141.6325 118.05) (end 141.55 118.05) (width 0.4) (layer F.Cu) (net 17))
 (segment (start 141.55 118.05) (end 140.5 118.05) (width 0.4) (layer F.Cu) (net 17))
 (segment (start 165 113.905) (end 165 114.493545) (width 0.4) (layer F.Cu) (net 18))
 (segment (start 165 114.493545) (end 161.493545 118) (width 0.4) (layer F.Cu) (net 18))
 (segment (start 161.493545 118) (end 157 118) (width 0.4) (layer F.Cu) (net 18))
 (segment (start 146 118) (end 157 118) (width 0.4) (layer B.Cu) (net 18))
 (via (at 157 118) (size 0.6) (drill 0.4) (layers F.Cu B.Cu) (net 18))
 (segment (start 144.5 119.5) (end 146 118) (width 0.4) (layer B.Cu) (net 18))
 (segment (start 144.05 119.95) (end 144.5 119.5) (width 0.4) (layer F.Cu) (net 18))
 (via (at 144.5 119.5) (size 0.6) (drill 0.4) (layers F.Cu B.Cu) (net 18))
 (segment (start 143.5 119.95) (end 144.05 119.95) (width 0.4) (layer F.Cu) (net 18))
 (segment (start 145.46 115.175) (end 145.46 116.09) (width 0.4) (layer F.Cu) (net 19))
 (segment (start 145.46 116.09) (end 143.5 118.05) (width 0.4) (layer F.Cu) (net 19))
 (segment (start 164 105) (end 164.007346 105) (width 0.6) (layer F.Cu) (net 20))
 (segment (start 164.007346 105) (end 165 105.992654) (width 0.6) (layer F.Cu) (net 20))
 (segment (start 165 105.992654) (end 165 108.825) (width 0.6) (layer F.Cu) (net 20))
 (segment (start 164.05 105) (end 164 105) (width 0.4) (layer F.Cu) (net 20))
 (segment (start 164.375 108.825) (end 165 108.825) (width 0.6) (layer F.Cu) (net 20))
 (segment (start 141.8 106.05) (end 139.55 106.05) (width 0.6) (layer F.Cu) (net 1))
 (segment (start 139.55 106.05) (end 139.5 106) (width 0.6) (layer F.Cu) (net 1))
 (segment (start 141.8 104.15) (end 142.605002 104.15) (width 0.6) (layer F.Cu) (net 1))
 (segment (start 142.605002 104.15) (end 142.830001 104.374999) (width 0.6) (layer F.Cu) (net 1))
 (segment (start 142.830001 104.374999) (end 142.830001 105.825001) (width 0.6) (layer F.Cu) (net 1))
 (segment (start 142.830001 105.825001) (end 142.605002 106.05) (width 0.6) (layer F.Cu) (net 1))
 (segment (start 142.605002 106.05) (end 141.8 106.05) (width 0.6) (layer F.Cu) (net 1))
 (segment (start 138.64884 110.10008) (end 138.90056 110.10008) (width 0.4) (layer F.Cu) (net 1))
 (segment (start 138.90056 110.10008) (end 139.5 110.69952) (width 0.4) (layer F.Cu) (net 1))
 (segment (start 139.5 110.69952) (end 139.80048 110.69952) (width 0.4) (layer F.Cu) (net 1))
 (segment (start 139.80048 110.69952) (end 140 110.5) (width 0.4) (layer F.Cu) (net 1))
 (segment (start 140 107.6) (end 140 110.5) (width 0.6) (layer F.Cu) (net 1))
 (segment (start 139.5 106) (end 139.5 107.1) (width 0.6) (layer F.Cu) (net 1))
 (segment (start 139.5 107.1) (end 140 107.6) (width 0.6) (layer F.Cu) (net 1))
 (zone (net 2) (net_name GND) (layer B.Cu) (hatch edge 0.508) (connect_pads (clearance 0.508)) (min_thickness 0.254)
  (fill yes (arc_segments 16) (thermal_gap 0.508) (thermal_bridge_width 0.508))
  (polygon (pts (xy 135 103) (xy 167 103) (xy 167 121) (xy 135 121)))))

